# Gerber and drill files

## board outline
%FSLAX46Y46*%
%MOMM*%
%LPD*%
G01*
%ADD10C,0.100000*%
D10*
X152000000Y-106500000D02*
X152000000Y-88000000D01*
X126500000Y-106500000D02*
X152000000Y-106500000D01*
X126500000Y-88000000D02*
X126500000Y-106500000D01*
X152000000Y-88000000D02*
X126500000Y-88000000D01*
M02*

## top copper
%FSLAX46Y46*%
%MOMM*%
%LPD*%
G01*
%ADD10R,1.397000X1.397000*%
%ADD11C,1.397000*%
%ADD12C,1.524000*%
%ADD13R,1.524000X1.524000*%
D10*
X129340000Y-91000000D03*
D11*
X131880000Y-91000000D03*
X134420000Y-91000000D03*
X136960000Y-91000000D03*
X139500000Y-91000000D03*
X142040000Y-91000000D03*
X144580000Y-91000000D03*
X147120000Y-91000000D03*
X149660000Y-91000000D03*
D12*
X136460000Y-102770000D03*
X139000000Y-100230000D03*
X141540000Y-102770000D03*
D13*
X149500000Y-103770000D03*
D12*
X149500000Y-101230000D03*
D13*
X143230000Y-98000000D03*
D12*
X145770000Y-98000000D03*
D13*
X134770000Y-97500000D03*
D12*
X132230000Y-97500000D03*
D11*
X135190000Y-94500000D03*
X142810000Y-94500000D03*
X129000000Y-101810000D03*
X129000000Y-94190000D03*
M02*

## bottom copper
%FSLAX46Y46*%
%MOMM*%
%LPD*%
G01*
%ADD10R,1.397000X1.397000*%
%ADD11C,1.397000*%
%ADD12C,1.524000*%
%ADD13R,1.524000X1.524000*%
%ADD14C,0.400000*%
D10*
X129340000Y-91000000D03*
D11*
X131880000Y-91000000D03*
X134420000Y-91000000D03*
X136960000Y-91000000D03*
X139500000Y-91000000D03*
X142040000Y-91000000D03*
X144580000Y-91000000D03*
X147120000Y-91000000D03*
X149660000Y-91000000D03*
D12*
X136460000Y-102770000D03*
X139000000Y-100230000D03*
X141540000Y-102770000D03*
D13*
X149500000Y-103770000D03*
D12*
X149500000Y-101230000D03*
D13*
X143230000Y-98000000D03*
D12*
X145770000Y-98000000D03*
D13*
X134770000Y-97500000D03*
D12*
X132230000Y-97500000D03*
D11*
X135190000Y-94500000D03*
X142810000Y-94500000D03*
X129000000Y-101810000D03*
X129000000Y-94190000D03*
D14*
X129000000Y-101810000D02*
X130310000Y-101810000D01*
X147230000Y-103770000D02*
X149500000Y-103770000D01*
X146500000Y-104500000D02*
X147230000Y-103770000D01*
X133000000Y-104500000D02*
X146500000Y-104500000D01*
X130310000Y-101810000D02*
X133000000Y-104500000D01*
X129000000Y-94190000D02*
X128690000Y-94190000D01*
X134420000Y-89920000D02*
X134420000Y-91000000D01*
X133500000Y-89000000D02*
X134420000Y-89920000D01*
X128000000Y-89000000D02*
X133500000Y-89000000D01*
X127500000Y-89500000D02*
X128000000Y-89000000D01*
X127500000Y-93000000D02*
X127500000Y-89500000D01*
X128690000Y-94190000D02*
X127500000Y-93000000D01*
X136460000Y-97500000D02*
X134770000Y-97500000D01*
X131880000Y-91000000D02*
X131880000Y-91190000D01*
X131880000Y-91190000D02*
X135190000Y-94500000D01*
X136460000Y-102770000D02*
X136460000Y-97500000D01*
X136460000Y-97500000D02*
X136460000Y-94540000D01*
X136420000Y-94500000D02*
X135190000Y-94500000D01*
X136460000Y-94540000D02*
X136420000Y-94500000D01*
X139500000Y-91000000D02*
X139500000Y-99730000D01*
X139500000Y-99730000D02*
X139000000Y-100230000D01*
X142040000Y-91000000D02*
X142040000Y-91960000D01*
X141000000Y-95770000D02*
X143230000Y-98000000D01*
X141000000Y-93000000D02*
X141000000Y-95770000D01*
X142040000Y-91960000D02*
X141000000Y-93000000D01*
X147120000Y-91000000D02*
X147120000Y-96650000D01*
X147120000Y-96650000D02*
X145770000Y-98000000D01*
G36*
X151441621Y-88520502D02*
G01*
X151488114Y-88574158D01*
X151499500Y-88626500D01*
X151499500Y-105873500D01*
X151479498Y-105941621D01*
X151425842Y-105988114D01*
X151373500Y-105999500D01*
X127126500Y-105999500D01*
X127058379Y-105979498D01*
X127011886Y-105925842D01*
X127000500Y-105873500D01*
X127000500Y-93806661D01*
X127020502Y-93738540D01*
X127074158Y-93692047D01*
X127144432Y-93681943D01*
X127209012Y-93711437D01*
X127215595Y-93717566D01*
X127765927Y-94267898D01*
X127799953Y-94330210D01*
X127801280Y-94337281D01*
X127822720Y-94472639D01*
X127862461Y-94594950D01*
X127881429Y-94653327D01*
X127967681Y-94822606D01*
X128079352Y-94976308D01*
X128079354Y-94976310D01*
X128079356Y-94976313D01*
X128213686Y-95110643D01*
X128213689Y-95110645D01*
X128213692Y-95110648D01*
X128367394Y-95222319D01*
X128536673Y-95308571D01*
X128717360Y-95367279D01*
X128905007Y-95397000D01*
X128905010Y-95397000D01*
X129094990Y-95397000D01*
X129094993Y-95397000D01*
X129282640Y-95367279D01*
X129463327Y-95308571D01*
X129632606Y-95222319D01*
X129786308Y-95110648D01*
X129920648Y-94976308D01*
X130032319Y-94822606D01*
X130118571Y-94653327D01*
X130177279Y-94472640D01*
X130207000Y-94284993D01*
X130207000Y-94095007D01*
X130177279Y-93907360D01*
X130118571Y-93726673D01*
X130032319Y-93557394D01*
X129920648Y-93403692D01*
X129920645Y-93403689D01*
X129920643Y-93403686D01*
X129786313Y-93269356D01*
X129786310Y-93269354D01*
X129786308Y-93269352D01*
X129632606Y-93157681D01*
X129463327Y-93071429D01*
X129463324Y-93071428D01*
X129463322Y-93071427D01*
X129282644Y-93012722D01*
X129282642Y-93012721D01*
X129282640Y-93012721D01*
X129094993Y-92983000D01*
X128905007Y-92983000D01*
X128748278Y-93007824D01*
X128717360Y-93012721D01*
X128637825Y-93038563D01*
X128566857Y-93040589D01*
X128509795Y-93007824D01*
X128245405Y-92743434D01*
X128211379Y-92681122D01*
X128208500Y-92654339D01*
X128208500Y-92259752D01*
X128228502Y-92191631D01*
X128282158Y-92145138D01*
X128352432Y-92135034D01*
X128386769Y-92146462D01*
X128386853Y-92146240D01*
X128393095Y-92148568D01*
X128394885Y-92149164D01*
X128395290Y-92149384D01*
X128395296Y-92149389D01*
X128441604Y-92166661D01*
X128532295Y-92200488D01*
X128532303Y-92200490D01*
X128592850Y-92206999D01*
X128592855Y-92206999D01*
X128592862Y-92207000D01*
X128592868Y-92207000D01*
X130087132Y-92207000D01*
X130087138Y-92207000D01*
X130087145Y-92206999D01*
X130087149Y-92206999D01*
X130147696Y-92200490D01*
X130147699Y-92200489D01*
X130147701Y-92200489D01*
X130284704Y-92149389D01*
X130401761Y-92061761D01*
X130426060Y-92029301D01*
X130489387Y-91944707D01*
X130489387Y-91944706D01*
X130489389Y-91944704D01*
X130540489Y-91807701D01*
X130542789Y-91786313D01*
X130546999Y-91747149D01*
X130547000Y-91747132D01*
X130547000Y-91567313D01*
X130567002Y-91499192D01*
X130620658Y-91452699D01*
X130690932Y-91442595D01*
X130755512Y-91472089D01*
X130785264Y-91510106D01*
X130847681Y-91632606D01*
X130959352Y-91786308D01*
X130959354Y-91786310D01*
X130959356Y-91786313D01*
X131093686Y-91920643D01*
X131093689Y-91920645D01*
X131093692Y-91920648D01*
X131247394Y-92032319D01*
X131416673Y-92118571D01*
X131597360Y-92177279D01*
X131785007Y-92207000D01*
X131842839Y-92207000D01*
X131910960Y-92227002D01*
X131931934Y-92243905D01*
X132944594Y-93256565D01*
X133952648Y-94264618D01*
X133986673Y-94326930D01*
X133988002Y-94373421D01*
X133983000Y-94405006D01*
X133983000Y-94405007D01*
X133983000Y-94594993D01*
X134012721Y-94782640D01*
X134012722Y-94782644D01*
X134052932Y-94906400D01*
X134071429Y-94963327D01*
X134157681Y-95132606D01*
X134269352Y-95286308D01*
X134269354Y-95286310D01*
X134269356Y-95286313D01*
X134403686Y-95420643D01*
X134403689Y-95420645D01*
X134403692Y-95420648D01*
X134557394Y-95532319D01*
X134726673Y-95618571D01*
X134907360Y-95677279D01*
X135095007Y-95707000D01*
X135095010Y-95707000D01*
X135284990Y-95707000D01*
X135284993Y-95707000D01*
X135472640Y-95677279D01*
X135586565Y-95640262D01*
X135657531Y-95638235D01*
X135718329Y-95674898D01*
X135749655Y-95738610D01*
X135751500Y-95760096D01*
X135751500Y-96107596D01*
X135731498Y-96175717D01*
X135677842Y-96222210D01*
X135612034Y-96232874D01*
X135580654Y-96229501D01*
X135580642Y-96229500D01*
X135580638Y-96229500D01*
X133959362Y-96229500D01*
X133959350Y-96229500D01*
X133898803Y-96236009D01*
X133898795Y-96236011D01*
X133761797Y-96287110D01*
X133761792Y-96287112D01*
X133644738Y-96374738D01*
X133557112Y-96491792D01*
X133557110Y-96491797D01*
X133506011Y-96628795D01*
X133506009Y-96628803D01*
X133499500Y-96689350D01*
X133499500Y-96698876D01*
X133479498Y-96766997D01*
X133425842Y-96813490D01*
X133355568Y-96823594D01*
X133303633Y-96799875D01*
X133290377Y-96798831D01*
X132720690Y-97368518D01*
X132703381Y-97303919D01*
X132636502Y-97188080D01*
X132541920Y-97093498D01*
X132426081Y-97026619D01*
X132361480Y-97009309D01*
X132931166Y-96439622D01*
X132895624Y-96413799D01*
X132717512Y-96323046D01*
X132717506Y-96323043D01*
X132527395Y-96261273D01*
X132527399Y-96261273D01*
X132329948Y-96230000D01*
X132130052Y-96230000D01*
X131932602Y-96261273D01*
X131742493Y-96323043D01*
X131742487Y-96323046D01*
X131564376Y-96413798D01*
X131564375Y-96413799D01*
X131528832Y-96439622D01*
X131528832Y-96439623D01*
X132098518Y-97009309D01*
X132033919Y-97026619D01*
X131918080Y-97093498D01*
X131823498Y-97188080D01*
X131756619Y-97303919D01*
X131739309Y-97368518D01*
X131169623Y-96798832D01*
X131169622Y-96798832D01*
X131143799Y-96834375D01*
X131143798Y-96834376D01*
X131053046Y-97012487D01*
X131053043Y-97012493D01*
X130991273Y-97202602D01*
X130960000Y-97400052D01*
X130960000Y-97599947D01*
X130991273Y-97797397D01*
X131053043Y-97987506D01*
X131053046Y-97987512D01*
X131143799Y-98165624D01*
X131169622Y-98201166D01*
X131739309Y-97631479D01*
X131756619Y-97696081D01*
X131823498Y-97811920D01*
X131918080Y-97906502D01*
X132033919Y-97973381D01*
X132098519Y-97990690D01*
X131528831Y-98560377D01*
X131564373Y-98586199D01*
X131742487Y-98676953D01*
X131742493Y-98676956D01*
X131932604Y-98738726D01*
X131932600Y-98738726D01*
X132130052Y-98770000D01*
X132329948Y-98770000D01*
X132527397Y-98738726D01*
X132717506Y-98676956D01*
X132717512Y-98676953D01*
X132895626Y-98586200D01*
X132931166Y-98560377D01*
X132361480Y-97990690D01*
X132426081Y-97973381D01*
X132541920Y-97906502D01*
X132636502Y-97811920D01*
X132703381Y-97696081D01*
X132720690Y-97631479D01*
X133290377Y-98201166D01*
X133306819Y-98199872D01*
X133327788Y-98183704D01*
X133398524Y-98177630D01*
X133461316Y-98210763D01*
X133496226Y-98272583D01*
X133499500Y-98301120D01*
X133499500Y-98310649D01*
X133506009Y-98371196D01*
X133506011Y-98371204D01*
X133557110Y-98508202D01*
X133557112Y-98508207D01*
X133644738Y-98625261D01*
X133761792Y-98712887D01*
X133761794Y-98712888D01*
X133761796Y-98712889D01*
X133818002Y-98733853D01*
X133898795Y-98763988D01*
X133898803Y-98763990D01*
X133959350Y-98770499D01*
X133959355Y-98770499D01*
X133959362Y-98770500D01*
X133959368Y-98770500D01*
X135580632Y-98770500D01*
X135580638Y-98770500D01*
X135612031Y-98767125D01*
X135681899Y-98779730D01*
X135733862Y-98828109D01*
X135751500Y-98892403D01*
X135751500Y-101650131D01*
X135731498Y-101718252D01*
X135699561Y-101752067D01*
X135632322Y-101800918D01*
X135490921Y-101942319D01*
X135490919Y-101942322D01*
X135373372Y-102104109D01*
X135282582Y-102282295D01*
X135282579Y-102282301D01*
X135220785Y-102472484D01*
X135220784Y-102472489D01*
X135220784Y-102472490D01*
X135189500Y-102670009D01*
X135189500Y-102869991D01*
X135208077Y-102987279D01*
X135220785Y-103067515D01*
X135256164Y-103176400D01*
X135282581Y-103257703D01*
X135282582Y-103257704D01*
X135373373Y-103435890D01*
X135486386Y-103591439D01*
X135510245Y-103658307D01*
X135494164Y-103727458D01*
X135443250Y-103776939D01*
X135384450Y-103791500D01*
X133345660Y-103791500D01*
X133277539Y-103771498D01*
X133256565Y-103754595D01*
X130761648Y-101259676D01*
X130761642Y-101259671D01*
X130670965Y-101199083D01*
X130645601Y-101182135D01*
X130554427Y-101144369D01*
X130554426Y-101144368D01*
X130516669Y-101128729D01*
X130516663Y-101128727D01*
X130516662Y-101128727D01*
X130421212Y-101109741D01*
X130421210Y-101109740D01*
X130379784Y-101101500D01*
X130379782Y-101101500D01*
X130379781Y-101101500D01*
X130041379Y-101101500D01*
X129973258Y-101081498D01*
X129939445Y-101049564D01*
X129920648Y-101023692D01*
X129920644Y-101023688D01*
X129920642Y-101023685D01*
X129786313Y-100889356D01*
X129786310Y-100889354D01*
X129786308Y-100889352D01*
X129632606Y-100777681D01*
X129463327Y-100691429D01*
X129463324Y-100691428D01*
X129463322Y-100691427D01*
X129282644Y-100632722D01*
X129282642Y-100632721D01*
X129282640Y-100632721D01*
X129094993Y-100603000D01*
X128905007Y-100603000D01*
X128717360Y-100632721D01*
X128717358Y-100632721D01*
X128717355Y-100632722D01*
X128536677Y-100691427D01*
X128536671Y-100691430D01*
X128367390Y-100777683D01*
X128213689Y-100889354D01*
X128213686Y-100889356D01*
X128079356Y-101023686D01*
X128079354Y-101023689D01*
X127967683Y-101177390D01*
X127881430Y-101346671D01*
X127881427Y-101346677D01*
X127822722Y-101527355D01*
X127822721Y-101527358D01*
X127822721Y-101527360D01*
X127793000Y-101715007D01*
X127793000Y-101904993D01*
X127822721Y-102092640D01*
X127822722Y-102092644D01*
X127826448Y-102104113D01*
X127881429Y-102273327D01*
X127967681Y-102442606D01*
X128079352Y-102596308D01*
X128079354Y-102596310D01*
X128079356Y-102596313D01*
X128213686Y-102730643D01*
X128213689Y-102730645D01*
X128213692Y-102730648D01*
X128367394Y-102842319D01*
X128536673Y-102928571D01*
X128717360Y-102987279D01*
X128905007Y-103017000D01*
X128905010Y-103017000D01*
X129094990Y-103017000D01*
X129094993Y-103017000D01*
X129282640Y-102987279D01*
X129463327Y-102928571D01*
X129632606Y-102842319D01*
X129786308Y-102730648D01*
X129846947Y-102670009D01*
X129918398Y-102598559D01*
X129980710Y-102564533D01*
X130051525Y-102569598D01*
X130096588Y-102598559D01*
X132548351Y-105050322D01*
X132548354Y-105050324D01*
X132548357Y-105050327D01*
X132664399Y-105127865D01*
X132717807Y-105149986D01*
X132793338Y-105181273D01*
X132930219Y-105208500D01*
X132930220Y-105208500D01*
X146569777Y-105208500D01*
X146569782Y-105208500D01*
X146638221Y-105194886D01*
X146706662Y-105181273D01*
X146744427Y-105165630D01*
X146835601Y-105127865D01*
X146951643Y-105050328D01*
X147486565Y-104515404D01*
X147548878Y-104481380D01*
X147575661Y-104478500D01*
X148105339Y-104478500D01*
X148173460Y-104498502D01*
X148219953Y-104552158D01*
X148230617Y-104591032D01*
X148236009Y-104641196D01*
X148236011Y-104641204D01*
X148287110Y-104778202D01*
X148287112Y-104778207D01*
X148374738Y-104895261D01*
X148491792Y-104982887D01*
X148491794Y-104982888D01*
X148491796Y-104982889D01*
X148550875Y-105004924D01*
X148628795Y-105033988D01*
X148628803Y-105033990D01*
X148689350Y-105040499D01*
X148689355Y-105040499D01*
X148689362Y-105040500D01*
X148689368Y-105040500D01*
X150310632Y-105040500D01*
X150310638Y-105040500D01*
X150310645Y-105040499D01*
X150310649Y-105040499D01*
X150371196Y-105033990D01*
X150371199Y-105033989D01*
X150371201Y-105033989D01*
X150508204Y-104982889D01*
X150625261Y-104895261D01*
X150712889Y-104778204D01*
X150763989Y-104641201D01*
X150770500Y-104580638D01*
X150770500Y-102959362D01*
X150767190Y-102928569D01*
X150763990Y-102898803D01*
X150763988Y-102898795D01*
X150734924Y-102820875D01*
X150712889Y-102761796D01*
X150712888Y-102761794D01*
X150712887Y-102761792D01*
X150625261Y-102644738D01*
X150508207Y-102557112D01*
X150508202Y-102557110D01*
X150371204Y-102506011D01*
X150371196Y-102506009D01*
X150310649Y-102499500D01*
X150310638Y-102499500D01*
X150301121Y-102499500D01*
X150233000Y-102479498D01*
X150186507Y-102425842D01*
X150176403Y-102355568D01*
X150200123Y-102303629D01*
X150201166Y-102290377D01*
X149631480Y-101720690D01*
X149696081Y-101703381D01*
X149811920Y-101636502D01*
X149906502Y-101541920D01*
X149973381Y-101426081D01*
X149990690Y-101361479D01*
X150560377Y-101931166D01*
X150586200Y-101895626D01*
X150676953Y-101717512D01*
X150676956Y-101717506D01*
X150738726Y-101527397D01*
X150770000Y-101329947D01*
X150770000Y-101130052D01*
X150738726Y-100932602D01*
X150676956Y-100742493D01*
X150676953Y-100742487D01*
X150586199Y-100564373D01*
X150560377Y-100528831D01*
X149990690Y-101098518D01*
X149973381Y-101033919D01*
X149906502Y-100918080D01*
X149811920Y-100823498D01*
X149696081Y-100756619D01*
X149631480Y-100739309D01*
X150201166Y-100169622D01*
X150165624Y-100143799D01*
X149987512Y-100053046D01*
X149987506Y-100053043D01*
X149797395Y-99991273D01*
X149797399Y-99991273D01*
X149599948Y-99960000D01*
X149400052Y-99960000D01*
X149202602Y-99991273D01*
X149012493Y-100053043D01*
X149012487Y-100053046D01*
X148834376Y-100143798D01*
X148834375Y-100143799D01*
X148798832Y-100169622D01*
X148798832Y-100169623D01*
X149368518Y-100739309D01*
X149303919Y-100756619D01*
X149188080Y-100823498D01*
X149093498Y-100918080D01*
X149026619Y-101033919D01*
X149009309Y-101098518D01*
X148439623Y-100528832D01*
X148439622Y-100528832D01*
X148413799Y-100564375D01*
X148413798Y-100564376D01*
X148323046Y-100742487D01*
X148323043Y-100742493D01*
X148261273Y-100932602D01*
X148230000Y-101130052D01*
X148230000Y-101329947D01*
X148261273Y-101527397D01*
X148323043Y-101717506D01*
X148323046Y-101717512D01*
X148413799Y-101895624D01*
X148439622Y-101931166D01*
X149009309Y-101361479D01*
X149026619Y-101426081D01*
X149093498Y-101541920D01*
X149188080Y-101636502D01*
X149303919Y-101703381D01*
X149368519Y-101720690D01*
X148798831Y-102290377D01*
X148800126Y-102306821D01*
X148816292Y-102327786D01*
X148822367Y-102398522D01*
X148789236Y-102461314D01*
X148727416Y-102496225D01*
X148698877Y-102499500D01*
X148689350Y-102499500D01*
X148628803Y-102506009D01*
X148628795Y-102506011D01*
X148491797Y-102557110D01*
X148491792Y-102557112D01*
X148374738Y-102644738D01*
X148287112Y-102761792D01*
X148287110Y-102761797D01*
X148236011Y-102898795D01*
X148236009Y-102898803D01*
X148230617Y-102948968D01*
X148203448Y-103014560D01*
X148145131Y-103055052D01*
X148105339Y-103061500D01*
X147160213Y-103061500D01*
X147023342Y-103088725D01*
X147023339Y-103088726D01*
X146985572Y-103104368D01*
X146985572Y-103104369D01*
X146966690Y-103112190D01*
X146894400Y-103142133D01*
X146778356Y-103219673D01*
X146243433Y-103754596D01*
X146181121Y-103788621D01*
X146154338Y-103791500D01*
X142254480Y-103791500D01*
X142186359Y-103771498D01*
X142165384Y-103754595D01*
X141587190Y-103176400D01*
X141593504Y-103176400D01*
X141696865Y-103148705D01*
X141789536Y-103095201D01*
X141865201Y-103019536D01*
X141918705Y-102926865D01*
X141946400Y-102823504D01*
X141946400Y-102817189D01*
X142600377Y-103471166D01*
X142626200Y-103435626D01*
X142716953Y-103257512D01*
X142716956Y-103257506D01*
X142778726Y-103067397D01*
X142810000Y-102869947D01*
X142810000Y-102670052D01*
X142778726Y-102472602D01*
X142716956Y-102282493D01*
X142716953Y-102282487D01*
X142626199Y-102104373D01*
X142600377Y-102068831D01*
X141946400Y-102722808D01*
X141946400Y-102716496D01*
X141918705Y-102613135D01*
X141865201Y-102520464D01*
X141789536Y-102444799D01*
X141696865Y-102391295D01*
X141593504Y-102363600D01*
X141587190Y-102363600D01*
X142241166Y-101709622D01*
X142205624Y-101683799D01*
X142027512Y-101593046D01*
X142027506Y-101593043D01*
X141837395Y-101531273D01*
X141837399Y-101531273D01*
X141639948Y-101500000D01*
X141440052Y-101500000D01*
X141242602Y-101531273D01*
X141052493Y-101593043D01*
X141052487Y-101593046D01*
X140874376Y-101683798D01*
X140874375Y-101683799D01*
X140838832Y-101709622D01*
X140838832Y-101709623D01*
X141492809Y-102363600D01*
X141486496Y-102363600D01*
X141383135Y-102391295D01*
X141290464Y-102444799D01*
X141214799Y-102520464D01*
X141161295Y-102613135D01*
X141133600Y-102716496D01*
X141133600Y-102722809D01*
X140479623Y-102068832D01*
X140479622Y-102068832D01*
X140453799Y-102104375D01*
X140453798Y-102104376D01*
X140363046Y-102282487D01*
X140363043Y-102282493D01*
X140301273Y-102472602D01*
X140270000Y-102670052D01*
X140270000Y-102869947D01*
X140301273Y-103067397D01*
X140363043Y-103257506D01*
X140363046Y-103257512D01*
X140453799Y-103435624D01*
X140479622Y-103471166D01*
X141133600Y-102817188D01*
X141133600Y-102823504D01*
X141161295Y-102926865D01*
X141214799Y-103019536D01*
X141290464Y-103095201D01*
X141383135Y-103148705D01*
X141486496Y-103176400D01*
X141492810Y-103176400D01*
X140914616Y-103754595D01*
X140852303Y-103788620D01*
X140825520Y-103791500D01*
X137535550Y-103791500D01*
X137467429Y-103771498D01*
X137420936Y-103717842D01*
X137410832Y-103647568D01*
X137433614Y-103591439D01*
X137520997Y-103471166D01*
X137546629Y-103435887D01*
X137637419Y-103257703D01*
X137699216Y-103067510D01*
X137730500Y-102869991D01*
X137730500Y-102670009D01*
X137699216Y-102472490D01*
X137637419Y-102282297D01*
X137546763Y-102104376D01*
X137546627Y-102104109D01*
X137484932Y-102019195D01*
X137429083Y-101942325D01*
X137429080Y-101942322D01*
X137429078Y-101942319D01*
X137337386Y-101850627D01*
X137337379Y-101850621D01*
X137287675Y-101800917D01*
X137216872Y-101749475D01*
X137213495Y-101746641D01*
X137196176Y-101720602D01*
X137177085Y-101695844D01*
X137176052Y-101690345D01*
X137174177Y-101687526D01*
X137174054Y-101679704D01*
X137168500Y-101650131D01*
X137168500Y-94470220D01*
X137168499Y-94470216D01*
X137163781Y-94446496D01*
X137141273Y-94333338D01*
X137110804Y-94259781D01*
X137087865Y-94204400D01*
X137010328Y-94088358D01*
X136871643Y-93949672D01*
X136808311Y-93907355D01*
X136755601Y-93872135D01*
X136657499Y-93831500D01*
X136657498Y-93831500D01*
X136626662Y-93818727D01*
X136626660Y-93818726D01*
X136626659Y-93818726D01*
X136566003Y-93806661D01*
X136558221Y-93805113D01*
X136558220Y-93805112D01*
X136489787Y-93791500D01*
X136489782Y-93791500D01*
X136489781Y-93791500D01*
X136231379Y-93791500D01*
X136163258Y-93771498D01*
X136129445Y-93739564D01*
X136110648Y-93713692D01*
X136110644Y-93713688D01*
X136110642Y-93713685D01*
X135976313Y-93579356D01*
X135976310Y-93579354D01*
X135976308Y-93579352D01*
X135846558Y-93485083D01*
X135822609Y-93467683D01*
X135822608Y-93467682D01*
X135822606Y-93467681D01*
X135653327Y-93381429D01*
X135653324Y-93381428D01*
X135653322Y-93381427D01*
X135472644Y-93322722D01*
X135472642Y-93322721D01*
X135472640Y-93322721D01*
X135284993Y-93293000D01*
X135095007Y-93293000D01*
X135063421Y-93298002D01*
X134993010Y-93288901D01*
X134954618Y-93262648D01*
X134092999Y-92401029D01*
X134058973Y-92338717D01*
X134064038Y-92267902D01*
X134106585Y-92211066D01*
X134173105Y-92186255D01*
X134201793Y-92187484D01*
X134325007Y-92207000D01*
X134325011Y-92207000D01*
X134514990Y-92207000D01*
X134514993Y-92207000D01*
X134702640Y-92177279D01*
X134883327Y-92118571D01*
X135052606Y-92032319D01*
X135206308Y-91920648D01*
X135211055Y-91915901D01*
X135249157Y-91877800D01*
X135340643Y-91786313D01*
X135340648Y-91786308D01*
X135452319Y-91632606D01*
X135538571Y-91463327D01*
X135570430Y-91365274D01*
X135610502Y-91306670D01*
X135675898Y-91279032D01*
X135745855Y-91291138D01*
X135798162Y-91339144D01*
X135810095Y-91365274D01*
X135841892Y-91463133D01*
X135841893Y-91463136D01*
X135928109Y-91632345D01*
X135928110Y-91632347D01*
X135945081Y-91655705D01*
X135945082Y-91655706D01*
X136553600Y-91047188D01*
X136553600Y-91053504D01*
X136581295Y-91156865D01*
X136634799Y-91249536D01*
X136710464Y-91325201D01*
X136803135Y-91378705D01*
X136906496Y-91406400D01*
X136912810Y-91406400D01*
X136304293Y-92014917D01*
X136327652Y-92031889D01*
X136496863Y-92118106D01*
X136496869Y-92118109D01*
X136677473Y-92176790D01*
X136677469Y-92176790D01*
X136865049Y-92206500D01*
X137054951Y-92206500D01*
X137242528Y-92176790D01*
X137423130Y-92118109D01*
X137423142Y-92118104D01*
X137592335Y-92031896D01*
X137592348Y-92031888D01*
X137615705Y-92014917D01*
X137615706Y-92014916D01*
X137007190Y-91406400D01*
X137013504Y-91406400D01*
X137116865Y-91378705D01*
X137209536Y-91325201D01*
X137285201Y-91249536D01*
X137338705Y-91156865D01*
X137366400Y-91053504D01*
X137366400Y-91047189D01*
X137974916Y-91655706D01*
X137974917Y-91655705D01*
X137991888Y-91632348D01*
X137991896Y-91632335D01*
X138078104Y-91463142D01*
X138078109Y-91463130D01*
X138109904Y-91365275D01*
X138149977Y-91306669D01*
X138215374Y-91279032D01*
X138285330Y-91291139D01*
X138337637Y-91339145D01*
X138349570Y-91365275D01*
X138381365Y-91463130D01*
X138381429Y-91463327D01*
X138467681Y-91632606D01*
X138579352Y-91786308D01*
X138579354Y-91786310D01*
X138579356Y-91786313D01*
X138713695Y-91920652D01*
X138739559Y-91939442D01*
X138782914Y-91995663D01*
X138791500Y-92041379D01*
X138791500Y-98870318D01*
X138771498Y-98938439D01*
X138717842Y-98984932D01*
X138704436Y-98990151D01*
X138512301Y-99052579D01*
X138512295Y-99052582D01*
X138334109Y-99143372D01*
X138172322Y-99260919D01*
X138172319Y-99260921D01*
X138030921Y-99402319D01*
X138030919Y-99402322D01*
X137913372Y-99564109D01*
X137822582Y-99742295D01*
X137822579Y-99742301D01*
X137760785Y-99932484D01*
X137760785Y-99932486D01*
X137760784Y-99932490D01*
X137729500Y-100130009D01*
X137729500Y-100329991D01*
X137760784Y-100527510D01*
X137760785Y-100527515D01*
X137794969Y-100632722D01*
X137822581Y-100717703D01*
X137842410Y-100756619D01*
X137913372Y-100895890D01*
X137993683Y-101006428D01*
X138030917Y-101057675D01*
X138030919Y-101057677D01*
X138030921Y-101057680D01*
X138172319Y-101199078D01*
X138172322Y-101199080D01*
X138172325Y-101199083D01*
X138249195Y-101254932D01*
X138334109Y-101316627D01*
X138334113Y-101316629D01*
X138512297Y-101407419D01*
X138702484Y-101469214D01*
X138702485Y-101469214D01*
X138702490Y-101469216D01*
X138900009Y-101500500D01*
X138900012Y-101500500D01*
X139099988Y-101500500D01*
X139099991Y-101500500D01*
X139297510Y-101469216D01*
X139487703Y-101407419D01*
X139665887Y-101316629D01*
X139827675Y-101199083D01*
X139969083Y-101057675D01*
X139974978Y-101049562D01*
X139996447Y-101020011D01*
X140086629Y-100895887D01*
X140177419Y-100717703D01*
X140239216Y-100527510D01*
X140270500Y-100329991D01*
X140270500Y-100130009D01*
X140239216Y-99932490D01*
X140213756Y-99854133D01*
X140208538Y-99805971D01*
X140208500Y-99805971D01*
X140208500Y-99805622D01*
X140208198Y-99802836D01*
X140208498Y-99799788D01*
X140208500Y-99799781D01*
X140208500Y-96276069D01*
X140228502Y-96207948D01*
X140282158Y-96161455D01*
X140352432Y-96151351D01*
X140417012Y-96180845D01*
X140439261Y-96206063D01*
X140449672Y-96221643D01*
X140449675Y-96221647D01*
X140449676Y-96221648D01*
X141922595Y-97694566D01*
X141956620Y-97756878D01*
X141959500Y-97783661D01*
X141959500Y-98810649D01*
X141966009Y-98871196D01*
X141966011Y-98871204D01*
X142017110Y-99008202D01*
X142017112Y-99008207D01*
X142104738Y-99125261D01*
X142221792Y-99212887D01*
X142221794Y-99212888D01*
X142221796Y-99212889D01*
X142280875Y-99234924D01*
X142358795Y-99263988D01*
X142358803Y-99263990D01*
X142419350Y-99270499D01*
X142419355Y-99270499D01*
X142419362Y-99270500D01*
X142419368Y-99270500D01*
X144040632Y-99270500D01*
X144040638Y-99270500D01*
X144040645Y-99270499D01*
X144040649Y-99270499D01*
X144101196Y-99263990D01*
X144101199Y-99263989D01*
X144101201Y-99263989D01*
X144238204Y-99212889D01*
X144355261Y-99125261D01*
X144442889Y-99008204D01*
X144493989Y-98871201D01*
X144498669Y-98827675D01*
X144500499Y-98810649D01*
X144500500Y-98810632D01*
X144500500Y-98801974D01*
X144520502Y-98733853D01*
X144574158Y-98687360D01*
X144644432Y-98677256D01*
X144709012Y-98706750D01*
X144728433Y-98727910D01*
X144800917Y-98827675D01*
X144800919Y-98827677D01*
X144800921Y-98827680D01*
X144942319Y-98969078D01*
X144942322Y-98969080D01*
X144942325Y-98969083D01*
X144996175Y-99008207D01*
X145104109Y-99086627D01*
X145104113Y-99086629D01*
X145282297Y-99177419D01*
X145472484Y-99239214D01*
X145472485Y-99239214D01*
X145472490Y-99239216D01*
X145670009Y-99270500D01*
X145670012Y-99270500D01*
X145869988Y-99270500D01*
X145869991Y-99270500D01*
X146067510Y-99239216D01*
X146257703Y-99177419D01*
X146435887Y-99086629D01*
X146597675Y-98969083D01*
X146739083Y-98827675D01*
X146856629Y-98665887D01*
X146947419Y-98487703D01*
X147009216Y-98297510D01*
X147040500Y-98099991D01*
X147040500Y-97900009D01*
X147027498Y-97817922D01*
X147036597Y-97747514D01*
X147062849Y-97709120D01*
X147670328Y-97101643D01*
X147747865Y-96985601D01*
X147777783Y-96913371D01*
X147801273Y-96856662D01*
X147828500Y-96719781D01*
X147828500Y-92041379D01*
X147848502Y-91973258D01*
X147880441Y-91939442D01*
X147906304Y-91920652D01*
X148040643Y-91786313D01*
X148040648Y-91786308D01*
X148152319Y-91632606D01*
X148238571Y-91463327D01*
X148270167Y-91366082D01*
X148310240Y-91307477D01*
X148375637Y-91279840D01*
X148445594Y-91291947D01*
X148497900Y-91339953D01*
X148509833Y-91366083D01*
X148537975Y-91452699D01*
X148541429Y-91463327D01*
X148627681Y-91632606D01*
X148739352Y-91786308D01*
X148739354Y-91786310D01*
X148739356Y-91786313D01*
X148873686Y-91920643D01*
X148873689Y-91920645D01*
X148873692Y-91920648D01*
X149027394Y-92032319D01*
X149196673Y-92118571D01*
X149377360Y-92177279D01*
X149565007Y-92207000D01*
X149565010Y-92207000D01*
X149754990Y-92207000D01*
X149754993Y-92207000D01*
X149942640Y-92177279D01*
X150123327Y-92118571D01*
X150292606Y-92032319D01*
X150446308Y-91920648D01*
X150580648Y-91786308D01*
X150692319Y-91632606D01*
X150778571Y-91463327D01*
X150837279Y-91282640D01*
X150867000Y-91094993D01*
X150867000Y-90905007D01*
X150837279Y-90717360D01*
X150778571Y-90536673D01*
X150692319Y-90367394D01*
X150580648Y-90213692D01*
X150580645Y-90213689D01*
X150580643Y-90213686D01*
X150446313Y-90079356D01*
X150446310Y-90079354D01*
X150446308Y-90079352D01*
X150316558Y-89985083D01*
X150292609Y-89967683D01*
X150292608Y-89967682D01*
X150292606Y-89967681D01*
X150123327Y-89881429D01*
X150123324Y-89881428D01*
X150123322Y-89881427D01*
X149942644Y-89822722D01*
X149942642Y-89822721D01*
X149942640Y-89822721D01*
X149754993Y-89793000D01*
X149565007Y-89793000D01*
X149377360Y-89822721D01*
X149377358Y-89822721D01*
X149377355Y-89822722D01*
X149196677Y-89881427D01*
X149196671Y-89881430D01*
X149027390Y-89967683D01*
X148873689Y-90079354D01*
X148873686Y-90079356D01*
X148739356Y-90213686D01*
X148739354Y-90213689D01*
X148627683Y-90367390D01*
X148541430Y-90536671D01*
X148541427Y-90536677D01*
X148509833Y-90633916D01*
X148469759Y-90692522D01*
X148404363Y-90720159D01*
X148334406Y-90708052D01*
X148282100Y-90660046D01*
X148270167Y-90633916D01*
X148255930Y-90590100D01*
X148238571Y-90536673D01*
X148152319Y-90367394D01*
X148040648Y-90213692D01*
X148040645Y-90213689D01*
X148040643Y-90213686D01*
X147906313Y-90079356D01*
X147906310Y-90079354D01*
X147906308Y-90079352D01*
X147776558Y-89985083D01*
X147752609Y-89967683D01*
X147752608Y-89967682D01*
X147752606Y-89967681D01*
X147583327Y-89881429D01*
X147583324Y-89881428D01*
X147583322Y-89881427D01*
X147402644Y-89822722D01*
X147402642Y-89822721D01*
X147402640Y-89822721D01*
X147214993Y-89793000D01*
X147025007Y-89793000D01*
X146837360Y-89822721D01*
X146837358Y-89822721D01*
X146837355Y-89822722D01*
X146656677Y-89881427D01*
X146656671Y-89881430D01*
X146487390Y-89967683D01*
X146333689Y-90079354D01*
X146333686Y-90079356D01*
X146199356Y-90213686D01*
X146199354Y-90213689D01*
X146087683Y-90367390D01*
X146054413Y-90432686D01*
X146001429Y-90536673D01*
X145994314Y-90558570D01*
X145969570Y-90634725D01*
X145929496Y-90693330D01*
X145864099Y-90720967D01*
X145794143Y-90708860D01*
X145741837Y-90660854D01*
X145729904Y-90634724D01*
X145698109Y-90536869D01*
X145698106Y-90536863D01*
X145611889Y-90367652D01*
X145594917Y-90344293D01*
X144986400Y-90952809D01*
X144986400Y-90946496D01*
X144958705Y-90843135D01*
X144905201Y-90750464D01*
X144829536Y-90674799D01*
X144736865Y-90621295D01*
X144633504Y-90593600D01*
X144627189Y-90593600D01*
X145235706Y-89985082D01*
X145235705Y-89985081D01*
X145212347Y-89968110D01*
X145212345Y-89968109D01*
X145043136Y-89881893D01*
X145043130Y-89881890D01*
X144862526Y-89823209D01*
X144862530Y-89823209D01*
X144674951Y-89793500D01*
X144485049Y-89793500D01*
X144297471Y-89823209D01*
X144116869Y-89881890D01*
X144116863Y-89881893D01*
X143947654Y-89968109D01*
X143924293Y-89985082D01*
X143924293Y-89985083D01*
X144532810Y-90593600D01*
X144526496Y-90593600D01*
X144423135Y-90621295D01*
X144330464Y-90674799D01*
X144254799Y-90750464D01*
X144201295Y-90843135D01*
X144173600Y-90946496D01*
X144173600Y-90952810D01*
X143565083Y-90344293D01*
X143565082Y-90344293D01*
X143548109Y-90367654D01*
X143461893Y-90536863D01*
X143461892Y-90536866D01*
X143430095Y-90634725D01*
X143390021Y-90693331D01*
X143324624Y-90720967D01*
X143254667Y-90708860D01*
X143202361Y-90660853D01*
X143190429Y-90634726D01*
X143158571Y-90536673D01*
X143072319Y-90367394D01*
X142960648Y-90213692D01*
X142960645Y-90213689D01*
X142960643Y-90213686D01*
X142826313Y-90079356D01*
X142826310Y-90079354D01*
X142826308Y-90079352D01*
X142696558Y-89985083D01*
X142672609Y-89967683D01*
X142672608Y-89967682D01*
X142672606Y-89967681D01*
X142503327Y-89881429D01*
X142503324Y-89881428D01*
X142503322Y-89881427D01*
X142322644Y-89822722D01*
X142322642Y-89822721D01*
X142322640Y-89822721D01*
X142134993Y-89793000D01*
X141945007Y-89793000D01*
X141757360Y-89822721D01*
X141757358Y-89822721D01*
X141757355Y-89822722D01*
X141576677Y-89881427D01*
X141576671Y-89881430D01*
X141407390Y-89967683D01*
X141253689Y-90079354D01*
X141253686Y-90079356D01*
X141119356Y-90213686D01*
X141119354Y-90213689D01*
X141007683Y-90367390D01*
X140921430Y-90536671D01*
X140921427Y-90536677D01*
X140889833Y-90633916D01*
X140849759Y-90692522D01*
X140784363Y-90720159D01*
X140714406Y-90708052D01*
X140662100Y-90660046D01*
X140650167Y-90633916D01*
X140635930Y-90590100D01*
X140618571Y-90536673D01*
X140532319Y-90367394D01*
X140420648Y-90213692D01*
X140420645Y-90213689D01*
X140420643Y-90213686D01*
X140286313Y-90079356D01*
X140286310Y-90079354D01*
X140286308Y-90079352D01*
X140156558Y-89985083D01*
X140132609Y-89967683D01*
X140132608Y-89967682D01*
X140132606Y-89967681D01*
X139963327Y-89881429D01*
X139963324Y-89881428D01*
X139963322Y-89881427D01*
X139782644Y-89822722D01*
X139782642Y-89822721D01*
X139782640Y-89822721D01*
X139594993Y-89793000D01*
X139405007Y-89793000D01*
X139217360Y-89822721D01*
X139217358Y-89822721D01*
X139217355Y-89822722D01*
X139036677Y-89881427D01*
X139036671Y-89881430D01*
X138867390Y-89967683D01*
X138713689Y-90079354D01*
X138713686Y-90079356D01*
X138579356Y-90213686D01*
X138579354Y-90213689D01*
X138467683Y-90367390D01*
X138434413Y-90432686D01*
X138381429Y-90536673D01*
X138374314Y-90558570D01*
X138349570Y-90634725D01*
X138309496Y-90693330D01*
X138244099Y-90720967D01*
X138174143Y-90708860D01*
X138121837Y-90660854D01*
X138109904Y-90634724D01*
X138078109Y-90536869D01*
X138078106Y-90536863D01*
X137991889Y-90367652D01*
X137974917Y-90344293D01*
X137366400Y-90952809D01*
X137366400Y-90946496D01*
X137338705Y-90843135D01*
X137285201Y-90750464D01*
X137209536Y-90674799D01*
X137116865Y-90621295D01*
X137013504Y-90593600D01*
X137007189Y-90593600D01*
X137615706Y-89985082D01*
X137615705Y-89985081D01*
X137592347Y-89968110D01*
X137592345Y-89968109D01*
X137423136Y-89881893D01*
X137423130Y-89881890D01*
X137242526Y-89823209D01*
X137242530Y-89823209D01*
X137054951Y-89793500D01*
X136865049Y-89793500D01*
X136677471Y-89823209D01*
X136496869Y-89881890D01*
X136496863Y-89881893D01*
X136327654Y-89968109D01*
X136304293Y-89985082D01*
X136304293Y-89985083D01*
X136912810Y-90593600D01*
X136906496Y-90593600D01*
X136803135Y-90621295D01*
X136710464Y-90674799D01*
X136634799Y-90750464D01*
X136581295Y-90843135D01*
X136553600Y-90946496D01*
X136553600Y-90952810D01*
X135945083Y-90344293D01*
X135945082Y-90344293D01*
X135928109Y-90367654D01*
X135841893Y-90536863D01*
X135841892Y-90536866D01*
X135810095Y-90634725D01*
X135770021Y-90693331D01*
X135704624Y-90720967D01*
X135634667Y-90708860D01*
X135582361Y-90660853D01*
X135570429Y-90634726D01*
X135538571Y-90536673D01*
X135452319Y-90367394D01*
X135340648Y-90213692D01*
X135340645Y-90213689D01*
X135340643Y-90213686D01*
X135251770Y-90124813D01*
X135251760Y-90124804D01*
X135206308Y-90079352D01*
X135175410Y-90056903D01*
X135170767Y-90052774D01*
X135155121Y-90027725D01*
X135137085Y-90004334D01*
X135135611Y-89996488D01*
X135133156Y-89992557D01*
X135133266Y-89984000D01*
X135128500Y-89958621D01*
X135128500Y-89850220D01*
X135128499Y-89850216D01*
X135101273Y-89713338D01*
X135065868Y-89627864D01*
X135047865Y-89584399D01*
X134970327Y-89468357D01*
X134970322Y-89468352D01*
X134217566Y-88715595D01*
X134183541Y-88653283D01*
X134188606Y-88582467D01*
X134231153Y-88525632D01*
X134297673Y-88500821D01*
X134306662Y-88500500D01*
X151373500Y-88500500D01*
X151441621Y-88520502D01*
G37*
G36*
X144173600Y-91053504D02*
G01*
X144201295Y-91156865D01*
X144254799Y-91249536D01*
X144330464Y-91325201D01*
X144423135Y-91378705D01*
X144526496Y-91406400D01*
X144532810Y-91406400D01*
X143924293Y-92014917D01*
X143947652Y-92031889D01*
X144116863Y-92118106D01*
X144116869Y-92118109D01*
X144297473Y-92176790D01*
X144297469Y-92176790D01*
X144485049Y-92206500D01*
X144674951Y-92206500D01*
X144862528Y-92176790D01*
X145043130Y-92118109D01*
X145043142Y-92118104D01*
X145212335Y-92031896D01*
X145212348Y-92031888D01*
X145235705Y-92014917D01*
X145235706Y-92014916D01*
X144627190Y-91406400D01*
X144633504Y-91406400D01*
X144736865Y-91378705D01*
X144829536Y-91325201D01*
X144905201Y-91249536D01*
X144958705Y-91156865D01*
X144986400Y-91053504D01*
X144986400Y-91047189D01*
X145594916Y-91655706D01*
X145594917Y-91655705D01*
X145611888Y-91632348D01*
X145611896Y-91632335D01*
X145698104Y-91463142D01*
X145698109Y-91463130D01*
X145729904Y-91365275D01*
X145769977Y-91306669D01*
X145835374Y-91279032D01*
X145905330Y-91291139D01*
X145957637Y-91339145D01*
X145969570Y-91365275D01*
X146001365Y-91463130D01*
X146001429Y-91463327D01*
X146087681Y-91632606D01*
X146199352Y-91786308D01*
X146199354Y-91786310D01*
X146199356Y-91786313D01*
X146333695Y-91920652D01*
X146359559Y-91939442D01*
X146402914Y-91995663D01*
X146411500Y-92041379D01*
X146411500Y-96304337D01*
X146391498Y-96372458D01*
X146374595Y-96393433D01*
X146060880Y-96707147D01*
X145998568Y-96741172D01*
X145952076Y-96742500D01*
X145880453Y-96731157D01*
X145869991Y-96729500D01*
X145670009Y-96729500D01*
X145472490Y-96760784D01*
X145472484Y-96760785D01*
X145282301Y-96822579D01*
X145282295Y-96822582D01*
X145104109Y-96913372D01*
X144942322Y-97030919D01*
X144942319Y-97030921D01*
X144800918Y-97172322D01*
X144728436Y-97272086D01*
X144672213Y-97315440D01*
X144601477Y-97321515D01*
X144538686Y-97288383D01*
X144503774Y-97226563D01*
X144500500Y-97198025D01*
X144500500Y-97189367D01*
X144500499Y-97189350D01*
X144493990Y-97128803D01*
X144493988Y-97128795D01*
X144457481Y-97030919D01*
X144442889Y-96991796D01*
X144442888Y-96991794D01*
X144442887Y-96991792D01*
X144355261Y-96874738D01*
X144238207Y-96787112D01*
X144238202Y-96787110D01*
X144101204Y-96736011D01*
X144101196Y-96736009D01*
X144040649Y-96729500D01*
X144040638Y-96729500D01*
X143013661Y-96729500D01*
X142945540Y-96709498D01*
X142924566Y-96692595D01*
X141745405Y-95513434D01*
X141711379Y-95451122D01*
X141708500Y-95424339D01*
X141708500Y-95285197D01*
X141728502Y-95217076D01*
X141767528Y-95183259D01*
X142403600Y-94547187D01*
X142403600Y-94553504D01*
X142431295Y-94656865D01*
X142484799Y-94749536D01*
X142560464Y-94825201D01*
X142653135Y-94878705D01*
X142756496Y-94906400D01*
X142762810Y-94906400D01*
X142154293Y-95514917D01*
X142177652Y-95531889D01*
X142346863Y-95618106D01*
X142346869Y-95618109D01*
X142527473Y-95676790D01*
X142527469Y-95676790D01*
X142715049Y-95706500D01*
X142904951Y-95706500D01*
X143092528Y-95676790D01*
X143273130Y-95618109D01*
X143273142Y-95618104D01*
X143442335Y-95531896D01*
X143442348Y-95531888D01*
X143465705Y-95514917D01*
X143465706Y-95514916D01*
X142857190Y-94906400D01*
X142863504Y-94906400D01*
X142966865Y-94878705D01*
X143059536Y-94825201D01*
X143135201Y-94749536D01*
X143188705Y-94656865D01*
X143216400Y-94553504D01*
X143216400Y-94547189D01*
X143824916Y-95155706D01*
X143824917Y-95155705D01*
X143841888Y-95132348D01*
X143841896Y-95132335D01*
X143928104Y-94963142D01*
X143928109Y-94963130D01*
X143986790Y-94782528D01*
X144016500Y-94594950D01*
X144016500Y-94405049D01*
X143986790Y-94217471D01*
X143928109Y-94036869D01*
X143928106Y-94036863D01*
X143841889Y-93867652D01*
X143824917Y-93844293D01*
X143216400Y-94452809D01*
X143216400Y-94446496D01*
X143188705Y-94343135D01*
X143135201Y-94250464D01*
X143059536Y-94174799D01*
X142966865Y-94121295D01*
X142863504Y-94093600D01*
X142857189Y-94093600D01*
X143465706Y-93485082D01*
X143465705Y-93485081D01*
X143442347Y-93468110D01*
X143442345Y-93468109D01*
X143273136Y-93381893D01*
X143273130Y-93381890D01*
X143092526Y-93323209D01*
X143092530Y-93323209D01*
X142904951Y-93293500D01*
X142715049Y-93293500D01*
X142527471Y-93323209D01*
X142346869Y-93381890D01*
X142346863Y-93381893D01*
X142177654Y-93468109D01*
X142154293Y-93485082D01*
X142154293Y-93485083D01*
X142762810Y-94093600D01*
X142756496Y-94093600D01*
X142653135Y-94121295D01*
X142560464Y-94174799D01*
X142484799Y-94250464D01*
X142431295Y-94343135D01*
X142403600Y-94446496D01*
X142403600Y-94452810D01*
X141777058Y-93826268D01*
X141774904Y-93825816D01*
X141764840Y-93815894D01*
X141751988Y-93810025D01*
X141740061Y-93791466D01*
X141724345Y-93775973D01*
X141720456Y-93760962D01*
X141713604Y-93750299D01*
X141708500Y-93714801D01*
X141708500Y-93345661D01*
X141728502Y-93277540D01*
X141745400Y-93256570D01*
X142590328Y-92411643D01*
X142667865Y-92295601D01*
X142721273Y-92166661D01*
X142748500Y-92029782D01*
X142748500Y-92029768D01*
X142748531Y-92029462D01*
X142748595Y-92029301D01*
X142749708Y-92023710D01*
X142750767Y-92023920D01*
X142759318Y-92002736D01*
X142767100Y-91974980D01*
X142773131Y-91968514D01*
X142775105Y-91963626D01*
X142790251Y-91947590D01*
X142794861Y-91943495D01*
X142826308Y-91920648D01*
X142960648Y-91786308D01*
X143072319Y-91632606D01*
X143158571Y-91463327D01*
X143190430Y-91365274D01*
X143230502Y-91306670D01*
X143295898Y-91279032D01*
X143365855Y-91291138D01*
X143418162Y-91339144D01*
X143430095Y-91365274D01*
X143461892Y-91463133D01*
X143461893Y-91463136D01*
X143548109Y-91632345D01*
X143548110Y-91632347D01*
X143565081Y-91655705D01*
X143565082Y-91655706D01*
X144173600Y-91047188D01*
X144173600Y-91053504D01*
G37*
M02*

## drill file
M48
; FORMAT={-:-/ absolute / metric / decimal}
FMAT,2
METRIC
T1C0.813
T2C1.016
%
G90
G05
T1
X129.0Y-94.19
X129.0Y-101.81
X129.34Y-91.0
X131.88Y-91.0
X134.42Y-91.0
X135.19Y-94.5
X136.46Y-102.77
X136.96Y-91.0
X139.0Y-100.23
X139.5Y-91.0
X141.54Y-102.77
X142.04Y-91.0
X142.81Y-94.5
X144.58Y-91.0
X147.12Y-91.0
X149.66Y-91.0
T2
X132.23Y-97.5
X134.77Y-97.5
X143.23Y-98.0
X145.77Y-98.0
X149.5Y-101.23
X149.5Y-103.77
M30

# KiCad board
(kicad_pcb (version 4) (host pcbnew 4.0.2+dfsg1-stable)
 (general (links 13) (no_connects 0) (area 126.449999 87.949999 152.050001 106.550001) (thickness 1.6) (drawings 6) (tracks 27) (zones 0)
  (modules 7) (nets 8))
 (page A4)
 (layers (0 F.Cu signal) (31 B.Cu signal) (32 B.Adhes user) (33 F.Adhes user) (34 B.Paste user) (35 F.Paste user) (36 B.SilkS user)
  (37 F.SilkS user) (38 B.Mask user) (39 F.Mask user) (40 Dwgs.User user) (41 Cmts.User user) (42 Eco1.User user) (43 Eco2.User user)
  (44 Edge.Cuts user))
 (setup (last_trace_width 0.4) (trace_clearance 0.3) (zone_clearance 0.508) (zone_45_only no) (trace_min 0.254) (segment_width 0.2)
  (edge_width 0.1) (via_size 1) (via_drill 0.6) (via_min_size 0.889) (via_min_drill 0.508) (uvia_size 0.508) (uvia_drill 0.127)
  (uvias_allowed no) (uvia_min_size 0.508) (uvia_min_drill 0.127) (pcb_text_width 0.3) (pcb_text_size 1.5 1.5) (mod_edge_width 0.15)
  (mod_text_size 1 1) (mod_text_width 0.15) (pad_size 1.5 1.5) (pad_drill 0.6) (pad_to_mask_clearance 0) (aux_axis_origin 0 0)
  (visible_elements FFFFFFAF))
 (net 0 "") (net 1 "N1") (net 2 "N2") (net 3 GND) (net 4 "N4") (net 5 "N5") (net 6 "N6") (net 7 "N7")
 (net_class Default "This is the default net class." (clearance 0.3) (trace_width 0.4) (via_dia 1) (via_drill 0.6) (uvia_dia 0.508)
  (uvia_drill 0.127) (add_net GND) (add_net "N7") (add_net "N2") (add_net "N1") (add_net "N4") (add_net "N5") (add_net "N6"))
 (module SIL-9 (layer F.Cu) (at 139.5 91)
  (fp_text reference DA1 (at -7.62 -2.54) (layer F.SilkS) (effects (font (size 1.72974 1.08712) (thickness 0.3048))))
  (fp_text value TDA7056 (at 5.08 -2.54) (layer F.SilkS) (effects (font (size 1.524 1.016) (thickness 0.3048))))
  (pad 1 thru_hole rect (at -10.16 0) (size 1.397 1.397) (drill 0.8128) (layers *.Cu *.Mask F.SilkS))
  (pad 2 thru_hole circle (at -7.62 0) (size 1.397 1.397) (drill 0.8128) (layers *.Cu *.Mask F.SilkS) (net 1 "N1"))
  (pad 3 thru_hole circle (at -5.08 0) (size 1.397 1.397) (drill 0.8128) (layers *.Cu *.Mask F.SilkS) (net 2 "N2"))
  (pad 4 thru_hole circle (at -2.54 0) (size 1.397 1.397) (drill 0.8128) (layers *.Cu *.Mask F.SilkS) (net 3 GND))
  (pad 5 thru_hole circle (at 0 0) (size 1.397 1.397) (drill 0.8128) (layers *.Cu *.Mask F.SilkS) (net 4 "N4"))
  (pad 6 thru_hole circle (at 2.54 0) (size 1.397 1.397) (drill 0.8128) (layers *.Cu *.Mask F.SilkS) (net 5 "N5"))
  (pad 7 thru_hole circle (at 5.08 0) (size 1.397 1.397) (drill 0.8128) (layers *.Cu *.Mask F.SilkS) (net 3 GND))
  (pad 8 thru_hole circle (at 7.62 0) (size 1.397 1.397) (drill 0.8128) (layers *.Cu *.Mask F.SilkS) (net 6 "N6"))
  (pad 9 thru_hole circle (at 10.16 0) (size 1.397 1.397) (drill 0.8128) (layers *.Cu *.Mask F.SilkS)))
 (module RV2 (layer F.Cu) (at 139 101.5) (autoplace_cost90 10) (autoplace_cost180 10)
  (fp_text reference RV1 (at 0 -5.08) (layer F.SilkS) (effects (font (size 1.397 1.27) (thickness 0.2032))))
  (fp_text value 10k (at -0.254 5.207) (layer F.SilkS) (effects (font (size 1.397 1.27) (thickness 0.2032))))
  (pad 1 thru_hole circle (at -2.54 1.27) (size 1.524 1.524) (drill 0.8128) (layers *.Cu *.Mask F.SilkS) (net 1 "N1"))
  (pad 2 thru_hole circle (at 0 -1.27) (size 1.524 1.524) (drill 0.8128) (layers *.Cu *.Mask F.SilkS) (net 4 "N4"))
  (pad 3 thru_hole circle (at 2.54 1.27) (size 1.524 1.524) (drill 0.8128) (layers *.Cu *.Mask F.SilkS) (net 3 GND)))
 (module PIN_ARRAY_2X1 (layer F.Cu) (at 149.5 102.5 90)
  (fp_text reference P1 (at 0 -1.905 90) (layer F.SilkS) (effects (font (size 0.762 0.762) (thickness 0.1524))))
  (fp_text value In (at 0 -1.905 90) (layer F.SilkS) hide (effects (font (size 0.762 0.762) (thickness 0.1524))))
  (pad 1 thru_hole rect (at -1.27 0 90) (size 1.524 1.524) (drill 1.016) (layers *.Cu *.Mask F.SilkS) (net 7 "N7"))
  (pad 2 thru_hole circle (at 1.27 0 90) (size 1.524 1.524) (drill 1.016) (layers *.Cu *.Mask F.SilkS) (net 3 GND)))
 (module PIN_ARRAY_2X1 (layer F.Cu) (at 144.5 98)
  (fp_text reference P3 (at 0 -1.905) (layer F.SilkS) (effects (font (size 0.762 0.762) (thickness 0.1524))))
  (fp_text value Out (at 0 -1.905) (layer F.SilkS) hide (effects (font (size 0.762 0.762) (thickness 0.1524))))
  (pad 1 thru_hole rect (at -1.27 0) (size 1.524 1.524) (drill 1.016) (layers *.Cu *.Mask F.SilkS) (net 5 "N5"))
  (pad 2 thru_hole circle (at 1.27 0) (size 1.524 1.524) (drill 1.016) (layers *.Cu *.Mask F.SilkS) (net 6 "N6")))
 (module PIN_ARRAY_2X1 (layer F.Cu) (at 133.5 97.5 180)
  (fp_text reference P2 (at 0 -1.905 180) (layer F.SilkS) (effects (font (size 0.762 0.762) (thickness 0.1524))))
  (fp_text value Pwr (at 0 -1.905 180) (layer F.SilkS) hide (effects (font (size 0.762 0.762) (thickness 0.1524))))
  (pad 1 thru_hole rect (at -1.27 0 180) (size 1.524 1.524) (drill 1.016) (layers *.Cu *.Mask F.SilkS) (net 1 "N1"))
  (pad 2 thru_hole circle (at 1.27 0 180) (size 1.524 1.524) (drill 1.016) (layers *.Cu *.Mask F.SilkS) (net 3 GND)))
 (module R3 (layer F.Cu) (at 139 94.5) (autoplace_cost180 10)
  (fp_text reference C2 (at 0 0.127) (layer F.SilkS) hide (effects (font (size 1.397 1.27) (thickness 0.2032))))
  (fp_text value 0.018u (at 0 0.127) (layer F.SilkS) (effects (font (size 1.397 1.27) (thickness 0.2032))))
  (pad 1 thru_hole circle (at -3.81 0) (size 1.397 1.397) (drill 0.8128) (layers *.Cu *.Mask F.SilkS) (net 1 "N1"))
  (pad 2 thru_hole circle (at 3.81 0) (size 1.397 1.397) (drill 0.8128) (layers *.Cu *.Mask F.SilkS) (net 3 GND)))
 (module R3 (layer F.Cu) (at 129 98 90) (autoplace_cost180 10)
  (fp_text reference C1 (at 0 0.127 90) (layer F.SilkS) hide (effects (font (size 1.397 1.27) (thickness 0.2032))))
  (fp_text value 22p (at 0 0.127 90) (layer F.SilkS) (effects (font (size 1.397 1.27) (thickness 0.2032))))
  (pad 1 thru_hole circle (at -3.81 0 90) (size 1.397 1.397) (drill 0.8128) (layers *.Cu *.Mask F.SilkS) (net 7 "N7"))
  (pad 2 thru_hole circle (at 3.81 0 90) (size 1.397 1.397) (drill 0.8128) (layers *.Cu *.Mask F.SilkS) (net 2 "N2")))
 (gr_line (start 152 106.5) (end 152 88) (angle 90) (layer Edge.Cuts) (width 0.1))
 (gr_line (start 126.5 106.5) (end 152 106.5) (angle 90) (layer Edge.Cuts) (width 0.1))
 (gr_line (start 126.5 88) (end 126.5 106.5) (angle 90) (layer Edge.Cuts) (width 0.1))
 (gr_line (start 152 88) (end 126.5 88) (angle 90) (layer Edge.Cuts) (width 0.1))
 (segment (start 129 101.81) (end 130.31 101.81) (width 0.4) (layer B.Cu) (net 7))
 (segment (start 147.23 103.77) (end 149.5 103.77) (width 0.4) (layer B.Cu) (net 7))
 (segment (start 146.5 104.5) (end 147.23 103.77) (width 0.4) (layer B.Cu) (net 7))
 (segment (start 133 104.5) (end 146.5 104.5) (width 0.4) (layer B.Cu) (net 7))
 (segment (start 130.31 101.81) (end 133 104.5) (width 0.4) (layer B.Cu) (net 7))
 (segment (start 129 94.19) (end 128.69 94.19) (width 0.4) (layer B.Cu) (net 2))
 (segment (start 134.42 89.92) (end 134.42 91) (width 0.4) (layer B.Cu) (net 2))
 (segment (start 133.5 89) (end 134.42 89.92) (width 0.4) (layer B.Cu) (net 2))
 (segment (start 128 89) (end 133.5 89) (width 0.4) (layer B.Cu) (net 2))
 (segment (start 127.5 89.5) (end 128 89) (width 0.4) (layer B.Cu) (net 2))
 (segment (start 127.5 93) (end 127.5 89.5) (width 0.4) (layer B.Cu) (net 2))
 (segment (start 128.69 94.19) (end 127.5 93) (width 0.4) (layer B.Cu) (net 2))
 (segment (start 136.46 97.5) (end 134.77 97.5) (width 0.4) (layer B.Cu) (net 1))
 (segment (start 131.88 91) (end 131.88 91.19) (width 0.4) (layer B.Cu) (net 1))
 (segment (start 131.88 91.19) (end 135.19 94.5) (width 0.4) (layer B.Cu) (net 1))
 (segment (start 136.46 102.77) (end 136.46 97.5) (width 0.4) (layer B.Cu) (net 1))
 (segment (start 136.46 97.5) (end 136.46 94.54) (width 0.4) (layer B.Cu) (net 1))
 (segment (start 136.42 94.5) (end 135.19 94.5) (width 0.4) (layer B.Cu) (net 1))
 (segment (start 136.46 94.54) (end 136.42 94.5) (width 0.4) (layer B.Cu) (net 1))
 (segment (start 139.5 91) (end 139.5 99.73) (width 0.4) (layer B.Cu) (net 4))
 (segment (start 139.5 99.73) (end 139 100.23) (width 0.4) (layer B.Cu) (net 4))
 (segment (start 142.04 91) (end 142.04 91.96) (width 0.4) (layer B.Cu) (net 5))
 (segment (start 141 95.77) (end 143.23 98) (width 0.4) (layer B.Cu) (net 5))
 (segment (start 141 93) (end 141 95.77) (width 0.4) (layer B.Cu) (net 5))
 (segment (start 142.04 91.96) (end 141 93) (width 0.4) (layer B.Cu) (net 5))
 (segment (start 147.12 91) (end 147.12 96.65) (width 0.4) (layer B.Cu) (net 6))
 (segment (start 147.12 96.65) (end 145.77 98) (width 0.4) (layer B.Cu) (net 6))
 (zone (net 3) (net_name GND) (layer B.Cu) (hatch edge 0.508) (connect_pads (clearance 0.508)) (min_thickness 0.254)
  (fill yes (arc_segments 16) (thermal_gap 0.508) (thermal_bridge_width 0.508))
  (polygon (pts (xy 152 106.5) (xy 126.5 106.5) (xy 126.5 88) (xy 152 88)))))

